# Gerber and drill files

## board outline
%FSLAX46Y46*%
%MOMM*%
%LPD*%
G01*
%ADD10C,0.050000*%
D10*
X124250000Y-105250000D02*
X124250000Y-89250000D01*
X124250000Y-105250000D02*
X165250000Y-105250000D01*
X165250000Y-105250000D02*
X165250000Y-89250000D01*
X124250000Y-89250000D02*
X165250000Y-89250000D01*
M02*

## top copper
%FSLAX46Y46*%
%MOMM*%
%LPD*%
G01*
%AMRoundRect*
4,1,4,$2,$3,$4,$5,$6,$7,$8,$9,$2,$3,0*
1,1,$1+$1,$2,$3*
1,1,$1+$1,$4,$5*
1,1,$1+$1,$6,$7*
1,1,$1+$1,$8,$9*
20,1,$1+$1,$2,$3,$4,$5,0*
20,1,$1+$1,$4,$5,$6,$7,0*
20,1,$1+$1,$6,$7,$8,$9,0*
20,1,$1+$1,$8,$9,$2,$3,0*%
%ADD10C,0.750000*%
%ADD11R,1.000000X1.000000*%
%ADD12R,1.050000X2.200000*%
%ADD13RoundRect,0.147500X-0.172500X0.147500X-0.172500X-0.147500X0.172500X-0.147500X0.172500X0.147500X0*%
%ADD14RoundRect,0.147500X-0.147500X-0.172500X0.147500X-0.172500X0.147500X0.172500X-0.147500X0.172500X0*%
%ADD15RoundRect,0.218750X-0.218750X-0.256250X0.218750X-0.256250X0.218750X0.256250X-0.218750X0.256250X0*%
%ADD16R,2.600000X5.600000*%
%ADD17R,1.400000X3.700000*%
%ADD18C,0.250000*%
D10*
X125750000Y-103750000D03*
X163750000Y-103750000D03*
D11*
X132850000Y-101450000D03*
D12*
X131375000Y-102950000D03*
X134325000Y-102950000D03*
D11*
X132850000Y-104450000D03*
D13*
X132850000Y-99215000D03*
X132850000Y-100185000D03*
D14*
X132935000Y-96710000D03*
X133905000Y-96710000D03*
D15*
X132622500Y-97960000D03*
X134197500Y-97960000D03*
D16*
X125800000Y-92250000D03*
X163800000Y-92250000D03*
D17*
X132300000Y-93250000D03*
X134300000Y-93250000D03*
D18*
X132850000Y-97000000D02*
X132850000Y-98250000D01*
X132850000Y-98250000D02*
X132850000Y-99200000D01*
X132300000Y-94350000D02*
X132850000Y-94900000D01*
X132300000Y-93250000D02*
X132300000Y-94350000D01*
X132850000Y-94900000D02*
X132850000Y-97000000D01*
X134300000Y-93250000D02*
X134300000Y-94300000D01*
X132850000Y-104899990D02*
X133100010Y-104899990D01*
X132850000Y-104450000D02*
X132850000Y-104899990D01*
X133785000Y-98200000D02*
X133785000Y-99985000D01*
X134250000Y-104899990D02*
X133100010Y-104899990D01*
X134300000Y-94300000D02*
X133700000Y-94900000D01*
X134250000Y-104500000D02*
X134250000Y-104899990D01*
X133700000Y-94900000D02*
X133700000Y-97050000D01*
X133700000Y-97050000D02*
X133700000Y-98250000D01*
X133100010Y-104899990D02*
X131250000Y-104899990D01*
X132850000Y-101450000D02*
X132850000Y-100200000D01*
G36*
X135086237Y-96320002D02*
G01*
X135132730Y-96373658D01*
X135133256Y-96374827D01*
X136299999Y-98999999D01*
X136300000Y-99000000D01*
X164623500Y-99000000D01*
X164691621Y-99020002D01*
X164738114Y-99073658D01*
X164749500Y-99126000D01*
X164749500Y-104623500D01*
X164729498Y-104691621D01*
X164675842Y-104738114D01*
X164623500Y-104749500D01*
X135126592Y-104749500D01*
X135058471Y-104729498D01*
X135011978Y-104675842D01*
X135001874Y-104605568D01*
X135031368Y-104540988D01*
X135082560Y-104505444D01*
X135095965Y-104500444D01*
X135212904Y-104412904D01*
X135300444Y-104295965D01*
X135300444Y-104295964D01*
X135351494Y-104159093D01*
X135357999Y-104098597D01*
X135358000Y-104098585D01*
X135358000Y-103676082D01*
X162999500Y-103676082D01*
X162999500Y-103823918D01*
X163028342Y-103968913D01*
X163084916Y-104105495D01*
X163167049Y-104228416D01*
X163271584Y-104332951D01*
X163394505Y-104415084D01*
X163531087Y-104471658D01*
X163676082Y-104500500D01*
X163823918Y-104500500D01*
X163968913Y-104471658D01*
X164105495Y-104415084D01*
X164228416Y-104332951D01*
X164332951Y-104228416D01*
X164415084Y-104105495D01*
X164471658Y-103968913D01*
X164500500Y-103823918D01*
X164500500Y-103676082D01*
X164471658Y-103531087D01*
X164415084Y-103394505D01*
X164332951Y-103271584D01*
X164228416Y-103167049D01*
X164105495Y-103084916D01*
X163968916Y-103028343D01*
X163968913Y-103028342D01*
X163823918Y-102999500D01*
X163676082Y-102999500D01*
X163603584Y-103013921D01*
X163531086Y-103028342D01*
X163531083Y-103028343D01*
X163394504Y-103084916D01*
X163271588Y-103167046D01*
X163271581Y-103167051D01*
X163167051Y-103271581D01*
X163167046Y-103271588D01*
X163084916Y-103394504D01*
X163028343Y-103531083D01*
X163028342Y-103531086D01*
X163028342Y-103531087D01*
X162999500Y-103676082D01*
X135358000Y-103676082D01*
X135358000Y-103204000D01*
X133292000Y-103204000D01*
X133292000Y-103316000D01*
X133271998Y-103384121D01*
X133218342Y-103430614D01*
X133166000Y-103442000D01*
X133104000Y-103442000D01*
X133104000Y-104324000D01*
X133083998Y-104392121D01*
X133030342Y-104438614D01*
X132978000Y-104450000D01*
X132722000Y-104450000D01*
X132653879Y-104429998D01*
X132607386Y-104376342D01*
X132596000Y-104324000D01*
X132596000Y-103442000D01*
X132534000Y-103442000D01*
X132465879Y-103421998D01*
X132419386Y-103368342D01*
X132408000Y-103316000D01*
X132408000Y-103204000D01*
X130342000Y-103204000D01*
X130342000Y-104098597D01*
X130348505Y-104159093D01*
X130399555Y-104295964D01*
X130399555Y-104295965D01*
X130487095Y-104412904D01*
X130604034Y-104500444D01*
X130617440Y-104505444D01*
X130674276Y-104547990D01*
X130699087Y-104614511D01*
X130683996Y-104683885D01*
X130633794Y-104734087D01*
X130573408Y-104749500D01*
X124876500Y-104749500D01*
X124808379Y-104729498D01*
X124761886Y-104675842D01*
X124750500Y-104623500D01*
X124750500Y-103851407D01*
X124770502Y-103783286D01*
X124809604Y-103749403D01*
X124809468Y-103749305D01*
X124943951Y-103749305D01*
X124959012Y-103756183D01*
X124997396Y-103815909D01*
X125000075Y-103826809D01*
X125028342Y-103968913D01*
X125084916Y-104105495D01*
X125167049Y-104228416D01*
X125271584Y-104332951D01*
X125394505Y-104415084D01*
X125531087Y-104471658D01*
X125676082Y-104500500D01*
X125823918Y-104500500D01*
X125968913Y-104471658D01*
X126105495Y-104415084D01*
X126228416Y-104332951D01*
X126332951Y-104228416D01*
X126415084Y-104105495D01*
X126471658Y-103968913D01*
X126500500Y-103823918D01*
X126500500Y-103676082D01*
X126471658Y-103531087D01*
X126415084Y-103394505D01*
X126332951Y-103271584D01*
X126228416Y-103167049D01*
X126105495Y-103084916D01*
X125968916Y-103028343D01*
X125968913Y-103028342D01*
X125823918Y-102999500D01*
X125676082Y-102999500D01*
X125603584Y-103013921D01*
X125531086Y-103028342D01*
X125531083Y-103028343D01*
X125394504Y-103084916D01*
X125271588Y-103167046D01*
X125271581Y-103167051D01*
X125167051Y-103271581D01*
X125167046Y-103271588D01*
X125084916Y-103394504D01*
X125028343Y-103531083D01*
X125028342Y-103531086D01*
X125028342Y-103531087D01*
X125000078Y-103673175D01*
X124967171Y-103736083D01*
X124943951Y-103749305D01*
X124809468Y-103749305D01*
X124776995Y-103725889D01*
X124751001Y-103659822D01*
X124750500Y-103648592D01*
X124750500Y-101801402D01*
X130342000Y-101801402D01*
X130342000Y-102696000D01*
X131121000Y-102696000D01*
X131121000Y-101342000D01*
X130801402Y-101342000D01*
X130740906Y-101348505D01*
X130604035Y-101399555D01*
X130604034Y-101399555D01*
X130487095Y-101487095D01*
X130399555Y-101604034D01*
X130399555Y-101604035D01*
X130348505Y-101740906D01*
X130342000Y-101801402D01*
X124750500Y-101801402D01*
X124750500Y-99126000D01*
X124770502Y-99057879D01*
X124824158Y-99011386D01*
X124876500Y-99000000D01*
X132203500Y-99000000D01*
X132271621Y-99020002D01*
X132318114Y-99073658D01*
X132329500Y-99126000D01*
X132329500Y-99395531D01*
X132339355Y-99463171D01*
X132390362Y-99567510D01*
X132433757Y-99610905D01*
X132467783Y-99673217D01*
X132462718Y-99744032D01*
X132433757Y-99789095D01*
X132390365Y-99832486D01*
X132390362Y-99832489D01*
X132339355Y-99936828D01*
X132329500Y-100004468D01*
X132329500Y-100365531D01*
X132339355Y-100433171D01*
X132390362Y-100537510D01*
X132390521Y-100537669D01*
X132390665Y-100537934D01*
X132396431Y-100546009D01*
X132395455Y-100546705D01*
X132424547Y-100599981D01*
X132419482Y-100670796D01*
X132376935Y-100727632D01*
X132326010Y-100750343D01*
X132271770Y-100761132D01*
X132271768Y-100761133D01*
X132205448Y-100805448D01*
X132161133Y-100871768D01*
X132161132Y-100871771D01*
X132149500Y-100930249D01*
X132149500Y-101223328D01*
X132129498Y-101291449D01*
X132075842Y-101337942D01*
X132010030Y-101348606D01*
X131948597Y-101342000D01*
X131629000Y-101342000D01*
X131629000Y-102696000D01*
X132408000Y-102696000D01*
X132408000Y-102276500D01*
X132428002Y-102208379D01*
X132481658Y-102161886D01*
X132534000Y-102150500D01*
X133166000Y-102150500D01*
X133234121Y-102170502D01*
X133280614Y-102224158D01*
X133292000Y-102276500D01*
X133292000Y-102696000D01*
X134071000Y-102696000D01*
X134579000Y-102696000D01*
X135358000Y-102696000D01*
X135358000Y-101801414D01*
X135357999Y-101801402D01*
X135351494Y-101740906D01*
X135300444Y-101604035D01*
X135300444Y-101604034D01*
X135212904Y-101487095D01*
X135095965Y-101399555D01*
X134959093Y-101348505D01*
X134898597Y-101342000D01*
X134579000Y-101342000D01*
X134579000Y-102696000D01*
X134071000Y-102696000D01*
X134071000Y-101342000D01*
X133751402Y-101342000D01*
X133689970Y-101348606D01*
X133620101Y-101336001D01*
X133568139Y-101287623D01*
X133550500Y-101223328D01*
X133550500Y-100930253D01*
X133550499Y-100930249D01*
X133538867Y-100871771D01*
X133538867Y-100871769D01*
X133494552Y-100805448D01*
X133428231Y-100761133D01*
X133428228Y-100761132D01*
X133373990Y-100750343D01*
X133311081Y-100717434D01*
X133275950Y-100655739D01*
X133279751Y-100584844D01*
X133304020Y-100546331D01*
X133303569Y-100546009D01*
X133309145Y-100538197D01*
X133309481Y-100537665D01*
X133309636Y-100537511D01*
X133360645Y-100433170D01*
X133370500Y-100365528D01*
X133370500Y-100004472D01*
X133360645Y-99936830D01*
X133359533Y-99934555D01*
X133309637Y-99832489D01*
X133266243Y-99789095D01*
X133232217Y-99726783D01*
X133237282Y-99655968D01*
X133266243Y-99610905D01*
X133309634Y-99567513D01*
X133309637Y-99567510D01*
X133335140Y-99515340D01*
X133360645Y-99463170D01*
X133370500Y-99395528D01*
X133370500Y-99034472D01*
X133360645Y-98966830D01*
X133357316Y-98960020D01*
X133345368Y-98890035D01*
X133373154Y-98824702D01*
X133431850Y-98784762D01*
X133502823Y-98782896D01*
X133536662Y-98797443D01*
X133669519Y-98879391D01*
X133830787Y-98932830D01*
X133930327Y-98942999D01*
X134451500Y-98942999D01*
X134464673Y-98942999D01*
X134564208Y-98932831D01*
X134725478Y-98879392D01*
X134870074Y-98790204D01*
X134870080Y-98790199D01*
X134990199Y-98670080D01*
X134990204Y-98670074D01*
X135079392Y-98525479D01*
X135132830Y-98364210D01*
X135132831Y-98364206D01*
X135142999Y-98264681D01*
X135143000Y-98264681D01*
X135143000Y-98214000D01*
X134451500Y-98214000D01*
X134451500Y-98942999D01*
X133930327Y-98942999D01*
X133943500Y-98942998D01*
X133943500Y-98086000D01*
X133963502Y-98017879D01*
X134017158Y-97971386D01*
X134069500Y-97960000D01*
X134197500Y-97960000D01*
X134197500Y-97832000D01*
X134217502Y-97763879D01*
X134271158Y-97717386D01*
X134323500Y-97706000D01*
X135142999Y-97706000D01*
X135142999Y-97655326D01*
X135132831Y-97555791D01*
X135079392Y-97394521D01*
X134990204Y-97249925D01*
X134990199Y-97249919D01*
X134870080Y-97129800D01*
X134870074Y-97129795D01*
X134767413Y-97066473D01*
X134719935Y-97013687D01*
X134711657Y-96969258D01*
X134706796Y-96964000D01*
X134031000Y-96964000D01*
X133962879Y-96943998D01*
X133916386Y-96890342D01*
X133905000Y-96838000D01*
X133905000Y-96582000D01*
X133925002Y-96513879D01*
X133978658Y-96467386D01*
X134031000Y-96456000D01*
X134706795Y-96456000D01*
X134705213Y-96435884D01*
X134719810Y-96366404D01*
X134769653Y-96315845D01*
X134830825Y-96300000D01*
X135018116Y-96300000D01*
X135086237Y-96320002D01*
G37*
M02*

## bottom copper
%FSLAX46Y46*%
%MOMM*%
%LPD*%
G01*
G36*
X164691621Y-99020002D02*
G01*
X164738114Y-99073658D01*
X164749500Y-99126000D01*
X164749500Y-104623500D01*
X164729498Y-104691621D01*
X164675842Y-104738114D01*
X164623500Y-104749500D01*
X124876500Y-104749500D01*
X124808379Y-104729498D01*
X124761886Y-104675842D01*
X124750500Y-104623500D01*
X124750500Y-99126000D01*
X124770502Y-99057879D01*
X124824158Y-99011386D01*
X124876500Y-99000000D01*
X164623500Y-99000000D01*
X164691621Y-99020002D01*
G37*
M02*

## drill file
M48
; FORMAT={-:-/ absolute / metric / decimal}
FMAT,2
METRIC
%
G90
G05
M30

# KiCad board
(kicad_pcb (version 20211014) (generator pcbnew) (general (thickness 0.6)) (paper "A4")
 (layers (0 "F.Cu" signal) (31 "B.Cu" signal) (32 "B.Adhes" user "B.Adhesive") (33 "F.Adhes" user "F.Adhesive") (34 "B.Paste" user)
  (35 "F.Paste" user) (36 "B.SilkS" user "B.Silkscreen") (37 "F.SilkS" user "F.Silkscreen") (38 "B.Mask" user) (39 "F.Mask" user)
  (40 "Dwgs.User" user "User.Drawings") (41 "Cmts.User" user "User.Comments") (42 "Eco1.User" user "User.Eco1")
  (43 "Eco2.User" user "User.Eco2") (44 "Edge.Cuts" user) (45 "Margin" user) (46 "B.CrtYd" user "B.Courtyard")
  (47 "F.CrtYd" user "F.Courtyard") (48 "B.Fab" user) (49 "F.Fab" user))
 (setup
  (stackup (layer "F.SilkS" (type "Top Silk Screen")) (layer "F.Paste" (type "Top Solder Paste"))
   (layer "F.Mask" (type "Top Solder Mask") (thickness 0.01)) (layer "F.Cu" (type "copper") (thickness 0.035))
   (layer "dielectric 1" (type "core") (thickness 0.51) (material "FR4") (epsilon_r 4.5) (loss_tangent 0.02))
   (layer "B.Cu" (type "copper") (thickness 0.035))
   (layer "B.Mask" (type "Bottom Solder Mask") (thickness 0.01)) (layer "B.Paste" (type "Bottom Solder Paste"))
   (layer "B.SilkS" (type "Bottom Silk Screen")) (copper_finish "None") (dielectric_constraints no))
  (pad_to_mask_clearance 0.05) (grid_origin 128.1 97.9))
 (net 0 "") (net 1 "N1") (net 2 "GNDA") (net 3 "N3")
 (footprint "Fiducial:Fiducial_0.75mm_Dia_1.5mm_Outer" (layer "F.Cu") (at 125.75 103.75)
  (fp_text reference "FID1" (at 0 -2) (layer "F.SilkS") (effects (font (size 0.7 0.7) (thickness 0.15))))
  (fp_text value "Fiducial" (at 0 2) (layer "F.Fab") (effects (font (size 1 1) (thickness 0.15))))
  (pad "" smd circle locked (at 0 0) (size 0.75 0.75) (layers "F.Cu" "F.Mask") (solder_mask_margin 0.375) (clearance 0.375)))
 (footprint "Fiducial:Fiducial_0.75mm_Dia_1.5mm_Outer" (layer "F.Cu") (at 163.75 103.75)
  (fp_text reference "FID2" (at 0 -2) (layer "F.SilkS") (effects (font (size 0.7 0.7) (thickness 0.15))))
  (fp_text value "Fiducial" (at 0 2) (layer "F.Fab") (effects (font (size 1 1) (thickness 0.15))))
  (pad "" smd circle locked (at 0 0) (size 0.75 0.75) (layers "F.Cu" "F.Mask") (solder_mask_margin 0.375) (clearance 0.375)))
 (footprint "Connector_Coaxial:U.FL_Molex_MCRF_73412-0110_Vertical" (layer "F.Cu") (at 132.85 102.95 180)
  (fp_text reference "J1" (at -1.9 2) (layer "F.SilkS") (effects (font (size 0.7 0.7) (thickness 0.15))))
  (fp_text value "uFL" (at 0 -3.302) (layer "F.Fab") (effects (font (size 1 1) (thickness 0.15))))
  (pad "1" smd rect locked (at 0 1.5 180) (size 1 1) (layers "F.Cu" "F.Paste" "F.Mask") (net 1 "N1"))
  (pad "2" smd rect locked (at 1.475 0 180) (size 1.05 2.2) (layers "F.Cu" "F.Paste" "F.Mask") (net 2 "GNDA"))
  (pad "2" smd rect locked (at -1.475 0 180) (size 1.05 2.2) (layers "F.Cu" "F.Paste" "F.Mask") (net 2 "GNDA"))
  (pad "2" smd rect locked (at 0 -1.5 180) (size 1 1) (layers "F.Cu" "F.Paste" "F.Mask") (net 2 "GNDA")))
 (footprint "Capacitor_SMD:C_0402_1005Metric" (layer "F.Cu") (at 132.85 99.7 -90)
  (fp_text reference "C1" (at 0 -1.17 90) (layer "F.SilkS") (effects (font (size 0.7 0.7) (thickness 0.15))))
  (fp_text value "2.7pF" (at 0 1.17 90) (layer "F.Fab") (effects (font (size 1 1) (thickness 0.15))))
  (pad "1" smd roundrect locked (at -0.485 0 270) (size 0.59 0.64) (layers "F.Cu" "F.Paste" "F.Mask") (roundrect_rratio 0.25) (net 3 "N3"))
  (pad "2" smd roundrect locked (at 0.485 0 270) (size 0.59 0.64) (layers "F.Cu" "F.Paste" "F.Mask") (roundrect_rratio 0.25) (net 1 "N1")))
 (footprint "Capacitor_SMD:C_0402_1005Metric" (layer "F.Cu") (at 133.42 96.71)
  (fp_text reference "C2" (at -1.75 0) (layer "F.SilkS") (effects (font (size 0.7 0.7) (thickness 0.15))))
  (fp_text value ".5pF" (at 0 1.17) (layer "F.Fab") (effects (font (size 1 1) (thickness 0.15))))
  (pad "1" smd roundrect locked (at -0.485 0) (size 0.59 0.64) (layers "F.Cu" "F.Paste" "F.Mask") (roundrect_rratio 0.25) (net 3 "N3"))
  (pad "2" smd roundrect locked (at 0.485 0) (size 0.59 0.64) (layers "F.Cu" "F.Paste" "F.Mask") (roundrect_rratio 0.25) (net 2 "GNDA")))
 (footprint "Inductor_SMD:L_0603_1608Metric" (layer "F.Cu") (at 133.41 97.96)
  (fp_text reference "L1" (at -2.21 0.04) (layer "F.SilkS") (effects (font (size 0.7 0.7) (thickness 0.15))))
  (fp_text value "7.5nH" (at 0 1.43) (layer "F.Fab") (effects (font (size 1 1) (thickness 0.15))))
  (pad "1" smd roundrect locked (at -0.7875 0) (size 0.875 0.95) (layers "F.Cu" "F.Paste" "F.Mask") (roundrect_rratio 0.25) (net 3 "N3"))
  (pad "2" smd roundrect locked (at 0.7875 0) (size 0.875 0.95) (layers "F.Cu" "F.Paste" "F.Mask") (roundrect_rratio 0.25) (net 2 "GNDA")))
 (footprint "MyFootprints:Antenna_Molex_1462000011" (layer "F.Cu") (at 145.3 92.25)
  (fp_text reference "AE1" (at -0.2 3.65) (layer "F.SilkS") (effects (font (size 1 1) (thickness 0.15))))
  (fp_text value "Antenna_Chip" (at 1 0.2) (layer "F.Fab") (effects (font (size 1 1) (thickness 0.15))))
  (pad "" smd rect locked (at -19.5 0) (size 2.6 5.6) (layers "F.Cu" "F.Paste" "F.Mask"))
  (pad "" smd rect locked (at 18.5 0) (size 2.6 5.6) (layers "F.Cu" "F.Paste" "F.Mask"))
  (pad "1" smd rect locked (at -13 1) (size 1.4 3.7) (layers "F.Cu" "F.Paste" "F.Mask") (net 3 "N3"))
  (pad "2" smd rect locked (at -11 1) (size 1.4 3.7) (layers "F.Cu" "F.Paste" "F.Mask") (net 2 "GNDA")))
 (gr_line (start 124.25 105.25) (end 124.25 89.25) (layer "Edge.Cuts") (width 0.05))
 (gr_line (start 124.25 105.25) (end 165.25 105.25) (layer "Edge.Cuts") (width 0.05))
 (gr_line (start 165.25 105.25) (end 165.25 89.25) (layer "Edge.Cuts") (width 0.05))
 (gr_line (start 124.25 89.25) (end 165.25 89.25) (layer "Edge.Cuts") (width 0.05))
 (segment (start 132.85 97) (end 132.85 98.25) (width 0.25) (layer "F.Cu") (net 3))
 (segment (start 132.85 98.25) (end 132.85 99.2) (width 0.25) (layer "F.Cu") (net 3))
 (segment (start 132.3 94.35) (end 132.85 94.9) (width 0.25) (layer "F.Cu") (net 3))
 (segment (start 132.3 93.25) (end 132.3 94.35) (width 0.25) (layer "F.Cu") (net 3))
 (segment (start 132.85 94.9) (end 132.85 97) (width 0.25) (layer "F.Cu") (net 3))
 (segment (start 134.3 93.25) (end 134.3 94.3) (width 0.25) (layer "F.Cu") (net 2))
 (segment (start 132.85 104.89999) (end 133.10001 104.89999) (width 0.25) (layer "F.Cu") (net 2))
 (segment (start 132.85 104.45) (end 132.85 104.89999) (width 0.25) (layer "F.Cu") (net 2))
 (segment (start 133.785 98.2) (end 133.785 99.985) (width 0.25) (layer "F.Cu") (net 2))
 (segment (start 134.25 104.89999) (end 133.10001 104.89999) (width 0.25) (layer "F.Cu") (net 2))
 (segment (start 134.3 94.3) (end 133.7 94.9) (width 0.25) (layer "F.Cu") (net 2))
 (segment (start 134.25 104.5) (end 134.25 104.89999) (width 0.25) (layer "F.Cu") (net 2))
 (segment (start 133.7 94.9) (end 133.7 97.05) (width 0.25) (layer "F.Cu") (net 2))
 (segment (start 133.7 97.05) (end 133.7 98.25) (width 0.25) (layer "F.Cu") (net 2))
 (segment (start 133.10001 104.89999) (end 131.25 104.89999) (width 0.25) (layer "F.Cu") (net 2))
 (segment (start 132.85 101.45) (end 132.85 100.2) (width 0.25) (layer "F.Cu") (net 1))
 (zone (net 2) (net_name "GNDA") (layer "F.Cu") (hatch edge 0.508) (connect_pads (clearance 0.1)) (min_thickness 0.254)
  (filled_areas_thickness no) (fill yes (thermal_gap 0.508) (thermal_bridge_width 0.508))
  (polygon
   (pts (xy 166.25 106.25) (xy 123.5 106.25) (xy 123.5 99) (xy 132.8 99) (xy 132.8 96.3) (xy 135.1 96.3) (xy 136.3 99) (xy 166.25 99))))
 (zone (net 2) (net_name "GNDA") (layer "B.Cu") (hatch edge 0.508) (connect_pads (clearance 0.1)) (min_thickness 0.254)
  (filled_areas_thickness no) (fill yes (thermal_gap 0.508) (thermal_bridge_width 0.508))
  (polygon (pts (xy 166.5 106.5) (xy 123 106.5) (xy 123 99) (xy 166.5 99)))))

